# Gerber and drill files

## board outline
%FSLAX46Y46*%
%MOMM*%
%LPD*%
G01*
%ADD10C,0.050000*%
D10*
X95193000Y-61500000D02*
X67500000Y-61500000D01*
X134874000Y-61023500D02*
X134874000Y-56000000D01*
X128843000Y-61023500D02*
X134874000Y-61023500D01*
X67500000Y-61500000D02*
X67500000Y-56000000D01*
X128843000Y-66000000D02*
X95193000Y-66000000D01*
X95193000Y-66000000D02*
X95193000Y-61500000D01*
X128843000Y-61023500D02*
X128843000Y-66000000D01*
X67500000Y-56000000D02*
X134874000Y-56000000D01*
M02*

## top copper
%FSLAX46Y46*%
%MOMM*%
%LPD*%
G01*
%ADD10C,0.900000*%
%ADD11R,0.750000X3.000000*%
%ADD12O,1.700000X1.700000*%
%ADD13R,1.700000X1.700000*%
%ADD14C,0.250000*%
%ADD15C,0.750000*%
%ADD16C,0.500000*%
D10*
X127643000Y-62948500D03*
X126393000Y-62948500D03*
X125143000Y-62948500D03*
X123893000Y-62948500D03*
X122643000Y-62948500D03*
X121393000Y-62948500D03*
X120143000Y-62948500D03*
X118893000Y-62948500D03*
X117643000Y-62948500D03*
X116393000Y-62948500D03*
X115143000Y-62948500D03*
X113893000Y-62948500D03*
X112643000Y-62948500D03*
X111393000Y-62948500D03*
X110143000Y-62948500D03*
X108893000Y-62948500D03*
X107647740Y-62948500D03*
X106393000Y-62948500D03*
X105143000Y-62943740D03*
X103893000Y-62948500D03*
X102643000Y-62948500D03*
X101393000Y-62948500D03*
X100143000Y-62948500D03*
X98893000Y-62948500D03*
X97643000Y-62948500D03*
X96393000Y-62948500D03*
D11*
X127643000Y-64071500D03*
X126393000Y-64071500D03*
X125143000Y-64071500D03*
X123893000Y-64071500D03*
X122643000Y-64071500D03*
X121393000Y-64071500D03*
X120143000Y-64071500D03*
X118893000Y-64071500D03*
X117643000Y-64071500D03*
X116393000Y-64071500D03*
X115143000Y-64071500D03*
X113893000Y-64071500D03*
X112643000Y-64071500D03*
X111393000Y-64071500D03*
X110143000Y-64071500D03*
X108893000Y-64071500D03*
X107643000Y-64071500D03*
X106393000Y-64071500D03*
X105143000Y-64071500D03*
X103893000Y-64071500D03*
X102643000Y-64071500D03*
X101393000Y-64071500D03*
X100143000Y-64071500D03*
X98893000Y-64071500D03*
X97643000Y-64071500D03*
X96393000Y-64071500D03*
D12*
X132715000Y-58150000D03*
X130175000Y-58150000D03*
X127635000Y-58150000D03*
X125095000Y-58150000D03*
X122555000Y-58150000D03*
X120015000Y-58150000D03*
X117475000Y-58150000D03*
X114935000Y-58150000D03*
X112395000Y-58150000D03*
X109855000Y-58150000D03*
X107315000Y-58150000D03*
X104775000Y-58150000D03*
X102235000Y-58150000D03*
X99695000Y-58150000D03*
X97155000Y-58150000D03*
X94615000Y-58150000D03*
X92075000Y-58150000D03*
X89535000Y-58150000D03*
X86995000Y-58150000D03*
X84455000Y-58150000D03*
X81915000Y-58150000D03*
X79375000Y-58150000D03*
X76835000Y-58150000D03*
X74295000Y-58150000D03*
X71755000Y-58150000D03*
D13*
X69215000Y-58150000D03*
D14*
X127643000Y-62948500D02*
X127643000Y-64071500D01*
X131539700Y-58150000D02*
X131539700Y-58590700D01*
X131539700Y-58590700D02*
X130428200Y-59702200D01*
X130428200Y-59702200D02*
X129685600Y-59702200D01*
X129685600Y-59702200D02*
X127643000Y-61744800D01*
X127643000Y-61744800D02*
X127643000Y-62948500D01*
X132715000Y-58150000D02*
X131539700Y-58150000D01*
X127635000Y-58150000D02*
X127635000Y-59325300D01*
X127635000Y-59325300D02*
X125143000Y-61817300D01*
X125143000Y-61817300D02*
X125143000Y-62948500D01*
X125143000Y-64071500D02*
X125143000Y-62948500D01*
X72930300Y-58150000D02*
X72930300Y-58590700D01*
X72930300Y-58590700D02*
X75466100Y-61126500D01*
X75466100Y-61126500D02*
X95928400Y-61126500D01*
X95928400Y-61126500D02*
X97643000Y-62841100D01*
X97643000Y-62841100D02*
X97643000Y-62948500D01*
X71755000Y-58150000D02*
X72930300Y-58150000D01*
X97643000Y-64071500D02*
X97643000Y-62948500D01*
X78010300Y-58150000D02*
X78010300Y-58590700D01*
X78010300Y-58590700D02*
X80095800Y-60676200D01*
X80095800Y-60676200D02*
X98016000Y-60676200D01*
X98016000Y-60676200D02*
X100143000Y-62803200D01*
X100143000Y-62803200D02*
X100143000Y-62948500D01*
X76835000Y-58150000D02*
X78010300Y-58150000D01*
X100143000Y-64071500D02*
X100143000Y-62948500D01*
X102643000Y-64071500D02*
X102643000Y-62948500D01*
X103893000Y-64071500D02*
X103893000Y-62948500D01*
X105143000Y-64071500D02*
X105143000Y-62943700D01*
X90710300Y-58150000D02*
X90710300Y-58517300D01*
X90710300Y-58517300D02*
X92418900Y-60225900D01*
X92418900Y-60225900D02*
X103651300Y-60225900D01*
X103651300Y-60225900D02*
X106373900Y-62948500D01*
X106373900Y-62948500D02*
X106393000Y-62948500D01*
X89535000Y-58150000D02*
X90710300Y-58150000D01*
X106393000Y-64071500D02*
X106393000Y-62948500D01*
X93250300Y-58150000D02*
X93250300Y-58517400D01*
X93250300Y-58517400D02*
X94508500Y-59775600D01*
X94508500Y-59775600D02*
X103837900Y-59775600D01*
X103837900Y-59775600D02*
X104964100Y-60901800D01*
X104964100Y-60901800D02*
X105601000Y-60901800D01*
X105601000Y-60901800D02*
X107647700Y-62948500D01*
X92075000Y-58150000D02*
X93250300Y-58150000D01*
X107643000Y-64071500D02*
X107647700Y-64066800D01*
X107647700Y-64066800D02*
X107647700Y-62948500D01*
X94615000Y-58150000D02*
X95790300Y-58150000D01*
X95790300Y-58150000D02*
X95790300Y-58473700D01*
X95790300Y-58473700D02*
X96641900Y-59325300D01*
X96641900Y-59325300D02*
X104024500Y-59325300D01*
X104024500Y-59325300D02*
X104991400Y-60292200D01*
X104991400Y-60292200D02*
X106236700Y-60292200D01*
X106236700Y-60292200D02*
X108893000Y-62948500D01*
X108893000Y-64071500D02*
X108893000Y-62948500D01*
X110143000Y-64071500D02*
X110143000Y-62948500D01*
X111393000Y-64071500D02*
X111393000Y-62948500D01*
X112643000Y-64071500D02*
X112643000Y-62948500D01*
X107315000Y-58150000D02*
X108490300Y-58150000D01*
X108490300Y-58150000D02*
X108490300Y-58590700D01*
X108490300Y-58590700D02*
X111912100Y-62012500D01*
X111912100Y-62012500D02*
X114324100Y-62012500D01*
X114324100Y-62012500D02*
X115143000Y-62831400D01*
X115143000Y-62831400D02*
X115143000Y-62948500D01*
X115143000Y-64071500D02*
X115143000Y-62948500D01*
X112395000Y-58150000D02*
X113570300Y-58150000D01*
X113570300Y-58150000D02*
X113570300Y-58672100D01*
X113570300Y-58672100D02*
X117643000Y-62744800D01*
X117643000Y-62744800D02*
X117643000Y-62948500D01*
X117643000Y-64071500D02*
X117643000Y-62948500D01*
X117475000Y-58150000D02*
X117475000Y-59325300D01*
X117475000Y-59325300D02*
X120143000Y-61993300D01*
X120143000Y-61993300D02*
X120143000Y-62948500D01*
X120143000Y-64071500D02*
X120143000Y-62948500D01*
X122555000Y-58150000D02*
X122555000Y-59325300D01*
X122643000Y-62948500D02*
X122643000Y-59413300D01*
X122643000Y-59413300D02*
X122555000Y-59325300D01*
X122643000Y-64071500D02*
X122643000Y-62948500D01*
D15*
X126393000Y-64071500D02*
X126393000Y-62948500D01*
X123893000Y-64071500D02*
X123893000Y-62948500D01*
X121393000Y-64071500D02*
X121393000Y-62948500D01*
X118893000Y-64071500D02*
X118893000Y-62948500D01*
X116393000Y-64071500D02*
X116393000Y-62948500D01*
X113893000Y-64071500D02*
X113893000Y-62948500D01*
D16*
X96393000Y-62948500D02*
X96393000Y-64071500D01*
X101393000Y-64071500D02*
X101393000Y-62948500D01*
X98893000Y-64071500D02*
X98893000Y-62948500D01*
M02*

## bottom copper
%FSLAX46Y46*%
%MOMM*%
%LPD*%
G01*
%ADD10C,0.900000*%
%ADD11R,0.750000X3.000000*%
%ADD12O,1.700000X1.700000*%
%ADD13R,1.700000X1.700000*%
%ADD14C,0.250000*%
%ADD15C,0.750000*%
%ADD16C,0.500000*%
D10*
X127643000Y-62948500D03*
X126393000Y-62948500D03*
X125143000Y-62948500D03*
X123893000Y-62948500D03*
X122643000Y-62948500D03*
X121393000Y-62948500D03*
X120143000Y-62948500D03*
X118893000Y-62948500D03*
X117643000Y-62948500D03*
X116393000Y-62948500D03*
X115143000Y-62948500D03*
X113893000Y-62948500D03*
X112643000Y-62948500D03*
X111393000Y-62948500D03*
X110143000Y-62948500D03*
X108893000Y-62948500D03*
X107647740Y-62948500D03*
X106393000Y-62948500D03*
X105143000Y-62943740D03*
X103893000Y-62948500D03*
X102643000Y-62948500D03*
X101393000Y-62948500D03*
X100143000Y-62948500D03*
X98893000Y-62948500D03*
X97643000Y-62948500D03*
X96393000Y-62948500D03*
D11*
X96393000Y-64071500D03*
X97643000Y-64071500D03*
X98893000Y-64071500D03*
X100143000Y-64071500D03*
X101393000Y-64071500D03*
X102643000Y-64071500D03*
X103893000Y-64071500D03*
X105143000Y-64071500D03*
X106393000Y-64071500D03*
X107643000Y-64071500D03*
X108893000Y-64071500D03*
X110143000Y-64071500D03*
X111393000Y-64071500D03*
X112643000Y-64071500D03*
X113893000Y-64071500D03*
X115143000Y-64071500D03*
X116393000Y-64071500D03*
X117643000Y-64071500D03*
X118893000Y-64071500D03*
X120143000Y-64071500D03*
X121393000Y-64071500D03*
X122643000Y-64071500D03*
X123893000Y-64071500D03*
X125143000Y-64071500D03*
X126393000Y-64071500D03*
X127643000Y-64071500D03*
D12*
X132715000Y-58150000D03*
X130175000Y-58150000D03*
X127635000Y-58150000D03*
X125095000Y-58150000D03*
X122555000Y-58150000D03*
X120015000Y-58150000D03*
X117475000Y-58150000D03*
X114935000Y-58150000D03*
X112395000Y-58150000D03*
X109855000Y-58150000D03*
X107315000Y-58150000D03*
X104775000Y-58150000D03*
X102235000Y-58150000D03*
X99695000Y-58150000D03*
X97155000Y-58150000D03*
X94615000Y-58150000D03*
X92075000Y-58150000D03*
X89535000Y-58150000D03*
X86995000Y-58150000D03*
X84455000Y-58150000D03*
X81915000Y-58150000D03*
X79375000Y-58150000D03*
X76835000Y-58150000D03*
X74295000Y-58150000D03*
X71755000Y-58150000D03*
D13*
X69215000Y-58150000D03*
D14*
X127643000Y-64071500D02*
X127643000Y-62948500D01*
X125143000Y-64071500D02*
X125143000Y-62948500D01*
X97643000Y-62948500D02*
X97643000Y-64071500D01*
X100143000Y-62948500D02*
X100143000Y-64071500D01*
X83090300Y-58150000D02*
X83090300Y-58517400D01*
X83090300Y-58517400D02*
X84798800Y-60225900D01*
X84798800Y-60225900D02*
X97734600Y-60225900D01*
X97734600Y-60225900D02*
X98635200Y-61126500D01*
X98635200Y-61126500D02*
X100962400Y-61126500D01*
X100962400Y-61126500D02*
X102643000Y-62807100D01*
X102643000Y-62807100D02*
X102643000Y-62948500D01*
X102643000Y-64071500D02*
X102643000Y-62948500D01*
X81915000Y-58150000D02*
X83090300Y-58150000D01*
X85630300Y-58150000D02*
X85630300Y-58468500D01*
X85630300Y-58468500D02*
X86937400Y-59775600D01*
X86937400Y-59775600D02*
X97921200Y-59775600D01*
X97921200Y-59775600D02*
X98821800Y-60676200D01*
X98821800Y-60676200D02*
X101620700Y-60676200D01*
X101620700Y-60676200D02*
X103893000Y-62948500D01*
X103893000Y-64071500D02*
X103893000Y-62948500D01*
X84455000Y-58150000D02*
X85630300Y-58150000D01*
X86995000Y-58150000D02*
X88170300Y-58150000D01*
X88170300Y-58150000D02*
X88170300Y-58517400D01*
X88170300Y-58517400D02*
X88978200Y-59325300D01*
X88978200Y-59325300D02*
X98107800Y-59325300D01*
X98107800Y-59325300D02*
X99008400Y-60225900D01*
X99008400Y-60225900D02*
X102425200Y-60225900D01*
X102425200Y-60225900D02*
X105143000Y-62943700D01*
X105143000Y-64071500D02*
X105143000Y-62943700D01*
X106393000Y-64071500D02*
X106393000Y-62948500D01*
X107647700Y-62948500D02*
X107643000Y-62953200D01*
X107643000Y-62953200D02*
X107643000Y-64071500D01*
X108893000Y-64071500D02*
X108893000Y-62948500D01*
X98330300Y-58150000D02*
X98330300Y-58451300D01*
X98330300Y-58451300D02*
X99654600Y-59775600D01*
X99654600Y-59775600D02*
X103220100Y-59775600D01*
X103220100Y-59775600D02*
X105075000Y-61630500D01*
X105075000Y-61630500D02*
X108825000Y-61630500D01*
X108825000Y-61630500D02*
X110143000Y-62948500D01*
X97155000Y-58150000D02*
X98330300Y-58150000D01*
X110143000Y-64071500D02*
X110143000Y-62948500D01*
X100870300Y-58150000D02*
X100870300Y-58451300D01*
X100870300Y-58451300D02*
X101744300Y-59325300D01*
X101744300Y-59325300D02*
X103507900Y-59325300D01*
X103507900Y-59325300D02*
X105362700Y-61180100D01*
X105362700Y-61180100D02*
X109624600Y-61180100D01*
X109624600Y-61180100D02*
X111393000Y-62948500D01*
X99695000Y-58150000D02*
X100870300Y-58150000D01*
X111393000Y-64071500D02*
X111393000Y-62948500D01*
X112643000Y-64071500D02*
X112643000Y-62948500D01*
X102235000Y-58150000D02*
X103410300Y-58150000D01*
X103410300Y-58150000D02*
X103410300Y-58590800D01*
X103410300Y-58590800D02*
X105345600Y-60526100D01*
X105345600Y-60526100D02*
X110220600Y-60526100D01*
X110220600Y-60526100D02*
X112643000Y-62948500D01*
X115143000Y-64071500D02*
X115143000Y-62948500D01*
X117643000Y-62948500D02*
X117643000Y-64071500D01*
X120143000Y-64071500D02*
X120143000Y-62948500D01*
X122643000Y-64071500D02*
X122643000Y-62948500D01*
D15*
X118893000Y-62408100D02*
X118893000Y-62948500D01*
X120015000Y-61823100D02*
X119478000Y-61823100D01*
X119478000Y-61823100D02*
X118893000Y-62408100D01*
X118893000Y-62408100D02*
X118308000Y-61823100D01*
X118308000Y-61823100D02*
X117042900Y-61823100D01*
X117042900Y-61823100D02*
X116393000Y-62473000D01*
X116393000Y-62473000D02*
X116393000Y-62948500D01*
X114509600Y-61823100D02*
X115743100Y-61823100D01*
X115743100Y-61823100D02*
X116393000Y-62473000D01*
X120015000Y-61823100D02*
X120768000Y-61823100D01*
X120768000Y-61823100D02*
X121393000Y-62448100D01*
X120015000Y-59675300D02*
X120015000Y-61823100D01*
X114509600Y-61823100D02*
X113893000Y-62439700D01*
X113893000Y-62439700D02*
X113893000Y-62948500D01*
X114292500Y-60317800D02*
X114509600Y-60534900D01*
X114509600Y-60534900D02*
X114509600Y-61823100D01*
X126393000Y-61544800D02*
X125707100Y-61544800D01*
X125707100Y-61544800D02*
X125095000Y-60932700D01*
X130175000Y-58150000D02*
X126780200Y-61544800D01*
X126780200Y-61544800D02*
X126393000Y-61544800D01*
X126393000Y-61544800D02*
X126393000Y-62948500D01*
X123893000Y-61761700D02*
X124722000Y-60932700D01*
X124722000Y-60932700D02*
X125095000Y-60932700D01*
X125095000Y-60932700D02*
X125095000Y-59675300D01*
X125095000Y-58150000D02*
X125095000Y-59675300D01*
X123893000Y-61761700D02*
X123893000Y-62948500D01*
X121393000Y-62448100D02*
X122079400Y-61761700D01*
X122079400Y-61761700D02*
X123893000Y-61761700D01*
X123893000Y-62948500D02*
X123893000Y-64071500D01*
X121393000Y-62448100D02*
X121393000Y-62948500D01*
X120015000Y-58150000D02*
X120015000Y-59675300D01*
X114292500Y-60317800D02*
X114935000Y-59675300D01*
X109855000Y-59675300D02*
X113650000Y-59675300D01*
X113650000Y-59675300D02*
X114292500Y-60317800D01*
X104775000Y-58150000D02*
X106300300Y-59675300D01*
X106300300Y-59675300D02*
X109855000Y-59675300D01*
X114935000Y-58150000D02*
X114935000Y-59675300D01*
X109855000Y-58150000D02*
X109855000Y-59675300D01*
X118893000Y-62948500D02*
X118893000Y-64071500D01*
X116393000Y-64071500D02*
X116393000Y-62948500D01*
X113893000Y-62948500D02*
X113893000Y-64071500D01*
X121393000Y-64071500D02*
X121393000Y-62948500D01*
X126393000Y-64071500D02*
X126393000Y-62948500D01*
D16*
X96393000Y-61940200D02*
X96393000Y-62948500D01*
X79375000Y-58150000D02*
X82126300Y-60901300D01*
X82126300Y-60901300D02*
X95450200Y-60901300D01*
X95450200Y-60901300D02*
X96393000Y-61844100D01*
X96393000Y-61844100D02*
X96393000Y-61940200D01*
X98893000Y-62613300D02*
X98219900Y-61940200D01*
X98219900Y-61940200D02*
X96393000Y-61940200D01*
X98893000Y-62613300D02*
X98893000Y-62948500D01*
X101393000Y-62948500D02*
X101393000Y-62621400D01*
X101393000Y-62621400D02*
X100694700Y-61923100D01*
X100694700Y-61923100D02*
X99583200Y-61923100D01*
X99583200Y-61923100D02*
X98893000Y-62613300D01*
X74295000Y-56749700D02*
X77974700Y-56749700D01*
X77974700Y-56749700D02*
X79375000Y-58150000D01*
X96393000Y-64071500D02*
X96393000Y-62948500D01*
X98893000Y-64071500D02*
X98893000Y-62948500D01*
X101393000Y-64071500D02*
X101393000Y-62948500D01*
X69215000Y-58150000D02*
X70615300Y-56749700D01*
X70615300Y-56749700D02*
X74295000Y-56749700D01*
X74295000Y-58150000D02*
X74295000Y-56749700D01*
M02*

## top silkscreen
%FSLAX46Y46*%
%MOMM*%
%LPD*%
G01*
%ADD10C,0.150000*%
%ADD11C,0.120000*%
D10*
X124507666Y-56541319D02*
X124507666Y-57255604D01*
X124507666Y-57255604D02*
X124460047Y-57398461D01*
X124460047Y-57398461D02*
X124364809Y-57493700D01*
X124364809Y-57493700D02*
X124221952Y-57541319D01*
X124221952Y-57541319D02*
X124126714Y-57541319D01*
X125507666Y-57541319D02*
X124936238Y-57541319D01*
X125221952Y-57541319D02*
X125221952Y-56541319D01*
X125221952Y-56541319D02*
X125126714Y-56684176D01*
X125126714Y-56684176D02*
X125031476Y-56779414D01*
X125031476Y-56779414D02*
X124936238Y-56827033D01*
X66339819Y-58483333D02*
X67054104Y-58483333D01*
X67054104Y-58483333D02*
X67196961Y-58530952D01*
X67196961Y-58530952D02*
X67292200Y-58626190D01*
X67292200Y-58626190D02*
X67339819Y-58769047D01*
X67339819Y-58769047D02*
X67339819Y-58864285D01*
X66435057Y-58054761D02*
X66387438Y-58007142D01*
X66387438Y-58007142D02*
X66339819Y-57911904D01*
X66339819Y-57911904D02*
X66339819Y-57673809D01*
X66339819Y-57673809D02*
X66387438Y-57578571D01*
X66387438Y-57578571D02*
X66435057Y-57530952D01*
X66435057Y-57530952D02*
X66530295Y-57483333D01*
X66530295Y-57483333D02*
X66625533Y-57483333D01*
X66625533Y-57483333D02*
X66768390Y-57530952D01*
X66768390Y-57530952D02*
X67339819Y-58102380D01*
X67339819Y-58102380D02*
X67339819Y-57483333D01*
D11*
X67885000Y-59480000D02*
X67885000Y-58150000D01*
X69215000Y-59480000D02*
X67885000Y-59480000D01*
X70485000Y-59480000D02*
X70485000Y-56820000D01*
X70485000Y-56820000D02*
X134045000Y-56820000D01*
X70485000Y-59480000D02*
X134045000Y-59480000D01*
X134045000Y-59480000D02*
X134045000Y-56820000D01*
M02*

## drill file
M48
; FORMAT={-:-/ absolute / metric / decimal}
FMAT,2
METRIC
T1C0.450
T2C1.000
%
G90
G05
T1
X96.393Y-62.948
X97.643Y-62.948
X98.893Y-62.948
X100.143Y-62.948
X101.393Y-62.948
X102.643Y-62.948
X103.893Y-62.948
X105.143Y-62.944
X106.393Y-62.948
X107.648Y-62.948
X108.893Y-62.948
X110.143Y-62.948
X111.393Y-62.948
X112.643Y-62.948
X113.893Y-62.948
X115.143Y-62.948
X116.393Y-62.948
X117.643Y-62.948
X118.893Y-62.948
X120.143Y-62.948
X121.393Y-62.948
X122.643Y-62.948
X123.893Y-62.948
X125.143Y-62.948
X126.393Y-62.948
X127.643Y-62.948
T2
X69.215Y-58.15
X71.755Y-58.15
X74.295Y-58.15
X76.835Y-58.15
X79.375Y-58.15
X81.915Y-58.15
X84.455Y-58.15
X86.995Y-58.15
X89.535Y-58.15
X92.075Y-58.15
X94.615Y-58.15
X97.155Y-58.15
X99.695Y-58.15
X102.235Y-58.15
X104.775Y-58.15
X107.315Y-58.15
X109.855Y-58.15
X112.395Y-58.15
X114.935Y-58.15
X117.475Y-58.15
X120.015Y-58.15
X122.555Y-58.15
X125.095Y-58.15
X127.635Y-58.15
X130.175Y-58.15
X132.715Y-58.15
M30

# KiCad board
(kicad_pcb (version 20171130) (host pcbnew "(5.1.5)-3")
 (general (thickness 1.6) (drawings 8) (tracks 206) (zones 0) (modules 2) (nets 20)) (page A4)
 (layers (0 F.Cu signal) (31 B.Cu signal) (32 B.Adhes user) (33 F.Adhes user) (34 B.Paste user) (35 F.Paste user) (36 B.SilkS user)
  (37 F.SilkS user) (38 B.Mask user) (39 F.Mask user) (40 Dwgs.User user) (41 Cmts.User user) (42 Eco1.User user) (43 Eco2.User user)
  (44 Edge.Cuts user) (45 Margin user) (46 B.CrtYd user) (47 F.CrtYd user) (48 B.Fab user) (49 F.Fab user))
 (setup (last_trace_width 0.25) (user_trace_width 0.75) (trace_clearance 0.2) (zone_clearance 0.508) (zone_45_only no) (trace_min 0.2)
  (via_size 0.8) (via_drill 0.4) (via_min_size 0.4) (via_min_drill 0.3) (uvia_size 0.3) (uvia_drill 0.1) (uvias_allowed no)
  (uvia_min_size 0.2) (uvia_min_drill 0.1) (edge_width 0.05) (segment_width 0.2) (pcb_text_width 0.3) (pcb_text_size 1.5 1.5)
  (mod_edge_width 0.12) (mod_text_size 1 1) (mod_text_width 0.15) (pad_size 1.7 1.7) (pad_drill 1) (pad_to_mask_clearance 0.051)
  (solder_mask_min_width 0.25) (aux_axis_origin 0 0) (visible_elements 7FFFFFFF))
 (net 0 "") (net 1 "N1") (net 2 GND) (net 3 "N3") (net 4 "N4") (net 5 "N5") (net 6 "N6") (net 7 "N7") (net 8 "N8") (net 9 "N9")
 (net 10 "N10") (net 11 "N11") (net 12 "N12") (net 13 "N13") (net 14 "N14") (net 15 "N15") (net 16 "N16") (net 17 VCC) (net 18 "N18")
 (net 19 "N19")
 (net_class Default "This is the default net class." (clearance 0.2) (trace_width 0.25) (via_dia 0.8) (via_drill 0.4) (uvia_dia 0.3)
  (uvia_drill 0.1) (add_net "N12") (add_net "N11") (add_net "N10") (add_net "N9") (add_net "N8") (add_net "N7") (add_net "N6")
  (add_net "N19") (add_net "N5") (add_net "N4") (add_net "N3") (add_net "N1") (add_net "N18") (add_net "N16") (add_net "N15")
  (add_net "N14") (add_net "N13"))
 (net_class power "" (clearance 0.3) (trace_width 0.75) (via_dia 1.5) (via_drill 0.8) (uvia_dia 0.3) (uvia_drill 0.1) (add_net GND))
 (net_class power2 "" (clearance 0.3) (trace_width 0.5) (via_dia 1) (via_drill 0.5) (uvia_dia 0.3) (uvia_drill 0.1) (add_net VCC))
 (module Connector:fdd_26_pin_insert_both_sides (layer F.Cu) (at 96.393 64.1985)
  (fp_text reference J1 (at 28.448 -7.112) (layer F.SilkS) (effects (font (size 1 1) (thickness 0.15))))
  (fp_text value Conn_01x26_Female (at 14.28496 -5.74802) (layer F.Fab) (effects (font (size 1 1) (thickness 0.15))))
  (pad 26 thru_hole circle (at 31.25 -1.25) (size 0.9 0.9) (drill 0.45) (layers *.Cu *.Mask) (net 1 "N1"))
  (pad 25 thru_hole circle (at 30 -1.25) (size 0.9 0.9) (drill 0.45) (layers *.Cu *.Mask) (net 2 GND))
  (pad 24 thru_hole circle (at 28.75 -1.25) (size 0.9 0.9) (drill 0.45) (layers *.Cu *.Mask) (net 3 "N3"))
  (pad 23 thru_hole circle (at 27.5 -1.25) (size 0.9 0.9) (drill 0.45) (layers *.Cu *.Mask) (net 2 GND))
  (pad 22 thru_hole circle (at 26.25 -1.25) (size 0.9 0.9) (drill 0.45) (layers *.Cu *.Mask) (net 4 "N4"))
  (pad 21 thru_hole circle (at 25 -1.25) (size 0.9 0.9) (drill 0.45) (layers *.Cu *.Mask) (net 2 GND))
  (pad 20 thru_hole circle (at 23.75 -1.25) (size 0.9 0.9) (drill 0.45) (layers *.Cu *.Mask) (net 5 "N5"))
  (pad 19 thru_hole circle (at 22.5 -1.25) (size 0.9 0.9) (drill 0.45) (layers *.Cu *.Mask) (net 2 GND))
  (pad 18 thru_hole circle (at 21.25 -1.25) (size 0.9 0.9) (drill 0.45) (layers *.Cu *.Mask) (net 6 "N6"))
  (pad 17 thru_hole circle (at 20 -1.25) (size 0.9 0.9) (drill 0.45) (layers *.Cu *.Mask) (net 2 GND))
  (pad 16 thru_hole circle (at 18.75 -1.25) (size 0.9 0.9) (drill 0.45) (layers *.Cu *.Mask) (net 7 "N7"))
  (pad 15 thru_hole circle (at 17.5 -1.25 90) (size 0.9 0.9) (drill 0.45) (layers *.Cu *.Mask) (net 2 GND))
  (pad 14 thru_hole circle (at 16.25 -1.25) (size 0.9 0.9) (drill 0.45) (layers *.Cu *.Mask) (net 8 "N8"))
  (pad 13 thru_hole circle (at 15 -1.25) (size 0.9 0.9) (drill 0.45) (layers *.Cu *.Mask) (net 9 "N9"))
  (pad 12 thru_hole circle (at 13.75 -1.25) (size 0.9 0.9) (drill 0.45) (layers *.Cu *.Mask) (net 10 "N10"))
  (pad 11 thru_hole circle (at 12.5 -1.25) (size 0.9 0.9) (drill 0.45) (layers *.Cu *.Mask) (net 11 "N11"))
  (pad 10 thru_hole circle (at 11.25474 -1.25) (size 0.9 0.9) (drill 0.45) (layers *.Cu *.Mask) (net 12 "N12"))
  (pad 9 thru_hole circle (at 10 -1.25) (size 0.9 0.9) (drill 0.45) (layers *.Cu *.Mask) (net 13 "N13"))
  (pad 8 thru_hole circle (at 8.75 -1.25476) (size 0.9 0.9) (drill 0.45) (layers *.Cu *.Mask) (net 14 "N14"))
  (pad 7 thru_hole circle (at 7.5 -1.25) (size 0.9 0.9) (drill 0.45) (layers *.Cu *.Mask) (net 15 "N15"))
  (pad 6 thru_hole circle (at 6.25 -1.25) (size 0.9 0.9) (drill 0.45) (layers *.Cu *.Mask) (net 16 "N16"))
  (pad 5 thru_hole circle (at 5 -1.25) (size 0.9 0.9) (drill 0.45) (layers *.Cu *.Mask) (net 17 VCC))
  (pad 4 thru_hole circle (at 3.75 -1.25) (size 0.9 0.9) (drill 0.45) (layers *.Cu *.Mask) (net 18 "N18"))
  (pad 3 thru_hole circle (at 2.5 -1.25) (size 0.9 0.9) (drill 0.45) (layers *.Cu *.Mask) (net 17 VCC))
  (pad 2 thru_hole circle (at 1.25 -1.25 90) (size 0.9 0.9) (drill 0.45) (layers *.Cu *.Mask) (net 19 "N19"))
  (pad 1 thru_hole circle (at 0 -1.25) (size 0.9 0.9) (drill 0.45) (layers *.Cu *.Mask) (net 17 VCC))
  (pad 26 connect rect (at 31.25 -0.127) (size 0.75 3) (layers F.Cu B.Mask) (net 1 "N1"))
  (pad 25 connect rect (at 30 -0.127) (size 0.75 3) (layers F.Cu B.Mask) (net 2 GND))
  (pad 24 connect rect (at 28.75 -0.127) (size 0.75 3) (layers F.Cu B.Mask) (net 3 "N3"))
  (pad 23 connect rect (at 27.5 -0.127) (size 0.75 3) (layers F.Cu B.Mask) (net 2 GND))
  (pad 22 connect rect (at 26.25 -0.127) (size 0.75 3) (layers F.Cu B.Mask) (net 4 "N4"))
  (pad 21 connect rect (at 25 -0.127) (size 0.75 3) (layers F.Cu B.Mask) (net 2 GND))
  (pad 20 connect rect (at 23.75 -0.127) (size 0.75 3) (layers F.Cu B.Mask) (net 5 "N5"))
  (pad 19 connect rect (at 22.5 -0.127) (size 0.75 3) (layers F.Cu B.Mask) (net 2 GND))
  (pad 18 connect rect (at 21.25 -0.127) (size 0.75 3) (layers F.Cu B.Mask) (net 6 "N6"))
  (pad 17 connect rect (at 20 -0.127) (size 0.75 3) (layers F.Cu B.Mask) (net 2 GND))
  (pad 16 connect rect (at 18.75 -0.127) (size 0.75 3) (layers F.Cu B.Mask) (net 7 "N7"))
  (pad 15 connect rect (at 17.5 -0.127) (size 0.75 3) (layers F.Cu B.Mask) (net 2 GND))
  (pad 14 connect rect (at 16.25 -0.127) (size 0.75 3) (layers F.Cu B.Mask) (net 8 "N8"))
  (pad 13 connect rect (at 15 -0.127) (size 0.75 3) (layers F.Cu B.Mask) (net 9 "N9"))
  (pad 12 connect rect (at 13.75 -0.127) (size 0.75 3) (layers F.Cu B.Mask) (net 10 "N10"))
  (pad 11 connect rect (at 12.5 -0.127) (size 0.75 3) (layers F.Cu B.Mask) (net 11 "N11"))
  (pad 10 connect rect (at 11.25 -0.127) (size 0.75 3) (layers F.Cu B.Mask) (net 12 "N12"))
  (pad 9 connect rect (at 10 -0.127) (size 0.75 3) (layers F.Cu B.Mask) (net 13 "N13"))
  (pad 8 connect rect (at 8.75 -0.127) (size 0.75 3) (layers F.Cu B.Mask) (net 14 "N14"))
  (pad 7 connect rect (at 7.5 -0.127) (size 0.75 3) (layers F.Cu B.Mask) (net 15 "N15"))
  (pad 6 connect rect (at 6.25 -0.127) (size 0.75 3) (layers F.Cu B.Mask) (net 16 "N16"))
  (pad 5 connect rect (at 5 -0.127) (size 0.75 3) (layers F.Cu B.Mask) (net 17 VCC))
  (pad 4 connect rect (at 3.75 -0.127) (size 0.75 3) (layers F.Cu B.Mask) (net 18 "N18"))
  (pad 3 connect rect (at 2.5 -0.127) (size 0.75 3) (layers F.Cu B.Mask) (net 17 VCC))
  (pad 2 connect rect (at 1.25 -0.127) (size 0.75 3) (layers F.Cu B.Mask) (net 19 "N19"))
  (pad 1 connect rect (at 0 -0.127) (size 0.75 3) (layers F.Cu B.Mask) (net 17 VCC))
  (pad 1 connect rect (at 0 -0.127) (size 0.75 3) (layers B.Cu B.Mask) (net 17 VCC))
  (pad 2 connect rect (at 1.25 -0.127) (size 0.75 3) (layers B.Cu B.Mask) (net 19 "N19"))
  (pad 3 connect rect (at 2.5 -0.127) (size 0.75 3) (layers B.Cu B.Mask) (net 17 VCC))
  (pad 4 connect rect (at 3.75 -0.127) (size 0.75 3) (layers B.Cu B.Mask) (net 18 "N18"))
  (pad 5 connect rect (at 5 -0.127) (size 0.75 3) (layers B.Cu B.Mask) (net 17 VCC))
  (pad 6 connect rect (at 6.25 -0.127) (size 0.75 3) (layers B.Cu B.Mask) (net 16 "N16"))
  (pad 7 connect rect (at 7.5 -0.127) (size 0.75 3) (layers B.Cu B.Mask) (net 15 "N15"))
  (pad 8 connect rect (at 8.75 -0.127) (size 0.75 3) (layers B.Cu B.Mask) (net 14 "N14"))
  (pad 9 connect rect (at 10 -0.127) (size 0.75 3) (layers B.Cu B.Mask) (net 13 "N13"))
  (pad 10 connect rect (at 11.25 -0.127) (size 0.75 3) (layers B.Cu B.Mask) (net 12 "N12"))
  (pad 11 connect rect (at 12.5 -0.127) (size 0.75 3) (layers B.Cu B.Mask) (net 11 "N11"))
  (pad 12 connect rect (at 13.75 -0.127) (size 0.75 3) (layers B.Cu B.Mask) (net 10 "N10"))
  (pad 13 connect rect (at 15 -0.127) (size 0.75 3) (layers B.Cu B.Mask) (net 9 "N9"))
  (pad 14 connect rect (at 16.25 -0.127) (size 0.75 3) (layers B.Cu B.Mask) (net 8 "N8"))
  (pad 15 connect rect (at 17.5 -0.127) (size 0.75 3) (layers B.Cu B.Mask) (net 2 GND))
  (pad 16 connect rect (at 18.75 -0.127) (size 0.75 3) (layers B.Cu B.Mask) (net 7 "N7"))
  (pad 17 connect rect (at 20 -0.127) (size 0.75 3) (layers B.Cu B.Mask) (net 2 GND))
  (pad 18 connect rect (at 21.25 -0.127) (size 0.75 3) (layers B.Cu B.Mask) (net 6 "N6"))
  (pad 19 connect rect (at 22.5 -0.127) (size 0.75 3) (layers B.Cu B.Mask) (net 2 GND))
  (pad 20 connect rect (at 23.75 -0.127) (size 0.75 3) (layers B.Cu B.Mask) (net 5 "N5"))
  (pad 21 connect rect (at 25 -0.127) (size 0.75 3) (layers B.Cu B.Mask) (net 2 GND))
  (pad 22 connect rect (at 26.25 -0.127) (size 0.75 3) (layers B.Cu B.Mask) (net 4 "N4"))
  (pad 23 connect rect (at 27.5 -0.127) (size 0.75 3) (layers B.Cu B.Mask) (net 2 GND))
  (pad 24 connect rect (at 28.75 -0.127) (size 0.75 3) (layers B.Cu B.Mask) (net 3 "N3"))
  (pad 25 connect rect (at 30 -0.127) (size 0.75 3) (layers B.Cu B.Mask) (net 2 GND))
  (pad 26 connect rect (at 31.25 -0.127) (size 0.75 3) (layers B.Cu B.Mask) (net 1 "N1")))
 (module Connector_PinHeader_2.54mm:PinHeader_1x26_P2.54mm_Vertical (layer F.Cu) (at 69.215 58.15 90)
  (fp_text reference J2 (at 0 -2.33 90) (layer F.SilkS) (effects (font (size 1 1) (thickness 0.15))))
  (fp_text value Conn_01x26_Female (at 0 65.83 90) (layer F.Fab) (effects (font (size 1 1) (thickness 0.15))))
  (fp_line (start -1.33 -1.33) (end 0 -1.33) (layer F.SilkS) (width 0.12))
  (fp_line (start -1.33 0) (end -1.33 -1.33) (layer F.SilkS) (width 0.12))
  (fp_line (start -1.33 1.27) (end 1.33 1.27) (layer F.SilkS) (width 0.12))
  (fp_line (start 1.33 1.27) (end 1.33 64.83) (layer F.SilkS) (width 0.12))
  (fp_line (start -1.33 1.27) (end -1.33 64.83) (layer F.SilkS) (width 0.12))
  (fp_line (start -1.33 64.83) (end 1.33 64.83) (layer F.SilkS) (width 0.12))
  (pad 26 thru_hole oval (at 0 63.5 90) (size 1.7 1.7) (drill 1) (layers *.Cu *.Mask) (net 1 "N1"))
  (pad 25 thru_hole oval (at 0 60.96 90) (size 1.7 1.7) (drill 1) (layers *.Cu *.Mask) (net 2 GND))
  (pad 24 thru_hole oval (at 0 58.42 90) (size 1.7 1.7) (drill 1) (layers *.Cu *.Mask) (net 3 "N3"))
  (pad 23 thru_hole oval (at 0 55.88 90) (size 1.7 1.7) (drill 1) (layers *.Cu *.Mask) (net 2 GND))
  (pad 22 thru_hole oval (at 0 53.34 90) (size 1.7 1.7) (drill 1) (layers *.Cu *.Mask) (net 4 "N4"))
  (pad 21 thru_hole oval (at 0 50.8 90) (size 1.7 1.7) (drill 1) (layers *.Cu *.Mask) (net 2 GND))
  (pad 20 thru_hole oval (at 0 48.26 90) (size 1.7 1.7) (drill 1) (layers *.Cu *.Mask) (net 5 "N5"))
  (pad 19 thru_hole oval (at 0 45.72 90) (size 1.7 1.7) (drill 1) (layers *.Cu *.Mask) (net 2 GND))
  (pad 18 thru_hole oval (at 0 43.18 90) (size 1.7 1.7) (drill 1) (layers *.Cu *.Mask) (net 6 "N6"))
  (pad 17 thru_hole oval (at 0 40.64 90) (size 1.7 1.7) (drill 1) (layers *.Cu *.Mask) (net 2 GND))
  (pad 16 thru_hole oval (at 0 38.1 90) (size 1.7 1.7) (drill 1) (layers *.Cu *.Mask) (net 7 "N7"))
  (pad 15 thru_hole oval (at 0 35.56 90) (size 1.7 1.7) (drill 1) (layers *.Cu *.Mask) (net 2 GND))
  (pad 14 thru_hole oval (at 0 33.02 90) (size 1.7 1.7) (drill 1) (layers *.Cu *.Mask) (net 8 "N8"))
  (pad 13 thru_hole oval (at 0 30.48 90) (size 1.7 1.7) (drill 1) (layers *.Cu *.Mask) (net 9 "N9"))
  (pad 12 thru_hole oval (at 0 27.94 90) (size 1.7 1.7) (drill 1) (layers *.Cu *.Mask) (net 10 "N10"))
  (pad 11 thru_hole oval (at 0 25.4 90) (size 1.7 1.7) (drill 1) (layers *.Cu *.Mask) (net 11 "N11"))
  (pad 10 thru_hole oval (at 0 22.86 90) (size 1.7 1.7) (drill 1) (layers *.Cu *.Mask) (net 12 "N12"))
  (pad 9 thru_hole oval (at 0 20.32 90) (size 1.7 1.7) (drill 1) (layers *.Cu *.Mask) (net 13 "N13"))
  (pad 8 thru_hole oval (at 0 17.78 90) (size 1.7 1.7) (drill 1) (layers *.Cu *.Mask) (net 14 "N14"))
  (pad 7 thru_hole oval (at 0 15.24 90) (size 1.7 1.7) (drill 1) (layers *.Cu *.Mask) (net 15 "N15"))
  (pad 6 thru_hole oval (at 0 12.7 90) (size 1.7 1.7) (drill 1) (layers *.Cu *.Mask) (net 16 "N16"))
  (pad 5 thru_hole oval (at 0 10.16 90) (size 1.7 1.7) (drill 1) (layers *.Cu *.Mask) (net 17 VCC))
  (pad 4 thru_hole oval (at 0 7.62 90) (size 1.7 1.7) (drill 1) (layers *.Cu *.Mask) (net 18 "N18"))
  (pad 3 thru_hole oval (at 0 5.08 90) (size 1.7 1.7) (drill 1) (layers *.Cu *.Mask) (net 17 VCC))
  (pad 2 thru_hole oval (at 0 2.54 90) (size 1.7 1.7) (drill 1) (layers *.Cu *.Mask) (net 19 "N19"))
  (pad 1 thru_hole rect (at 0 0 90) (size 1.7 1.7) (drill 1) (layers *.Cu *.Mask) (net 17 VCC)))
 (gr_line (start 95.193 61.5) (end 67.5 61.5) (layer Edge.Cuts) (width 0.05))
 (gr_line (start 134.874 61.0235) (end 134.874 56) (layer Edge.Cuts) (width 0.05))
 (gr_line (start 128.843 61.0235) (end 134.874 61.0235) (layer Edge.Cuts) (width 0.05))
 (gr_line (start 67.5 61.5) (end 67.5 56) (layer Edge.Cuts) (width 0.05))
 (gr_line (start 128.843 66) (end 95.193 66) (layer Edge.Cuts) (width 0.05))
 (gr_line (start 95.193 66) (end 95.193 61.5) (layer Edge.Cuts) (width 0.05))
 (gr_line (start 128.843 61.0235) (end 128.843 66) (layer Edge.Cuts) (width 0.05))
 (gr_line (start 67.5 56) (end 134.874 56) (layer Edge.Cuts) (width 0.05))
 (segment (start 127.643 62.9485) (end 127.643 64.0715) (width 0.25) (layer F.Cu) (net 1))
 (segment (start 131.5397 58.15) (end 131.5397 58.5907) (width 0.25) (layer F.Cu) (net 1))
 (segment (start 131.5397 58.5907) (end 130.4282 59.7022) (width 0.25) (layer F.Cu) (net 1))
 (segment (start 130.4282 59.7022) (end 129.6856 59.7022) (width 0.25) (layer F.Cu) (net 1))
 (segment (start 129.6856 59.7022) (end 127.643 61.7448) (width 0.25) (layer F.Cu) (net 1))
 (segment (start 127.643 61.7448) (end 127.643 62.9485) (width 0.25) (layer F.Cu) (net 1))
 (segment (start 127.643 64.0715) (end 127.643 62.9485) (width 0.25) (layer B.Cu) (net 1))
 (segment (start 132.715 58.15) (end 131.5397 58.15) (width 0.25) (layer F.Cu) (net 1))
 (segment (start 127.635 58.15) (end 127.635 59.3253) (width 0.25) (layer F.Cu) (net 3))
 (segment (start 127.635 59.3253) (end 125.143 61.8173) (width 0.25) (layer F.Cu) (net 3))
 (segment (start 125.143 61.8173) (end 125.143 62.9485) (width 0.25) (layer F.Cu) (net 3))
 (segment (start 125.143 64.0715) (end 125.143 62.9485) (width 0.25) (layer B.Cu) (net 3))
 (segment (start 125.143 64.0715) (end 125.143 62.9485) (width 0.25) (layer F.Cu) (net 3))
 (segment (start 72.9303 58.15) (end 72.9303 58.5907) (width 0.25) (layer F.Cu) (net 19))
 (segment (start 72.9303 58.5907) (end 75.4661 61.1265) (width 0.25) (layer F.Cu) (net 19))
 (segment (start 75.4661 61.1265) (end 95.9284 61.1265) (width 0.25) (layer F.Cu) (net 19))
 (segment (start 95.9284 61.1265) (end 97.643 62.8411) (width 0.25) (layer F.Cu) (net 19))
 (segment (start 97.643 62.8411) (end 97.643 62.9485) (width 0.25) (layer F.Cu) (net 19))
 (segment (start 71.755 58.15) (end 72.9303 58.15) (width 0.25) (layer F.Cu) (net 19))
 (segment (start 97.643 62.9485) (end 97.643 64.0715) (width 0.25) (layer B.Cu) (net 19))
 (segment (start 97.643 64.0715) (end 97.643 62.9485) (width 0.25) (layer F.Cu) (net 19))
 (segment (start 78.0103 58.15) (end 78.0103 58.5907) (width 0.25) (layer F.Cu) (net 18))
 (segment (start 78.0103 58.5907) (end 80.0958 60.6762) (width 0.25) (layer F.Cu) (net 18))
 (segment (start 80.0958 60.6762) (end 98.016 60.6762) (width 0.25) (layer F.Cu) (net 18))
 (segment (start 98.016 60.6762) (end 100.143 62.8032) (width 0.25) (layer F.Cu) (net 18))
 (segment (start 100.143 62.8032) (end 100.143 62.9485) (width 0.25) (layer F.Cu) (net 18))
 (segment (start 76.835 58.15) (end 78.0103 58.15) (width 0.25) (layer F.Cu) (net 18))
 (segment (start 100.143 62.9485) (end 100.143 64.0715) (width 0.25) (layer B.Cu) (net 18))
 (segment (start 100.143 64.0715) (end 100.143 62.9485) (width 0.25) (layer F.Cu) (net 18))
 (segment (start 83.0903 58.15) (end 83.0903 58.5174) (width 0.25) (layer B.Cu) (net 16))
 (segment (start 83.0903 58.5174) (end 84.7988 60.2259) (width 0.25) (layer B.Cu) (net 16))
 (segment (start 84.7988 60.2259) (end 97.7346 60.2259) (width 0.25) (layer B.Cu) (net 16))
 (segment (start 97.7346 60.2259) (end 98.6352 61.1265) (width 0.25) (layer B.Cu) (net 16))
 (segment (start 98.6352 61.1265) (end 100.9624 61.1265) (width 0.25) (layer B.Cu) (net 16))
 (segment (start 100.9624 61.1265) (end 102.643 62.8071) (width 0.25) (layer B.Cu) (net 16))
 (segment (start 102.643 62.8071) (end 102.643 62.9485) (width 0.25) (layer B.Cu) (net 16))
 (segment (start 102.643 64.0715) (end 102.643 62.9485) (width 0.25) (layer F.Cu) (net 16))
 (segment (start 102.643 64.0715) (end 102.643 62.9485) (width 0.25) (layer B.Cu) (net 16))
 (segment (start 81.915 58.15) (end 83.0903 58.15) (width 0.25) (layer B.Cu) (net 16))
 (segment (start 85.6303 58.15) (end 85.6303 58.4685) (width 0.25) (layer B.Cu) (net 15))
 (segment (start 85.6303 58.4685) (end 86.9374 59.7756) (width 0.25) (layer B.Cu) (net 15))
 (segment (start 86.9374 59.7756) (end 97.9212 59.7756) (width 0.25) (layer B.Cu) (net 15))
 (segment (start 97.9212 59.7756) (end 98.8218 60.6762) (width 0.25) (layer B.Cu) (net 15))
 (segment (start 98.8218 60.6762) (end 101.6207 60.6762) (width 0.25) (layer B.Cu) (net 15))
 (segment (start 101.6207 60.6762) (end 103.893 62.9485) (width 0.25) (layer B.Cu) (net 15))
 (segment (start 103.893 64.0715) (end 103.893 62.9485) (width 0.25) (layer F.Cu) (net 15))
 (segment (start 103.893 64.0715) (end 103.893 62.9485) (width 0.25) (layer B.Cu) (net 15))
 (segment (start 84.455 58.15) (end 85.6303 58.15) (width 0.25) (layer B.Cu) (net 15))
 (segment (start 86.995 58.15) (end 88.1703 58.15) (width 0.25) (layer B.Cu) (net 14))
 (segment (start 88.1703 58.15) (end 88.1703 58.5174) (width 0.25) (layer B.Cu) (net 14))
 (segment (start 88.1703 58.5174) (end 88.9782 59.3253) (width 0.25) (layer B.Cu) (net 14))
 (segment (start 88.9782 59.3253) (end 98.1078 59.3253) (width 0.25) (layer B.Cu) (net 14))
 (segment (start 98.1078 59.3253) (end 99.0084 60.2259) (width 0.25) (layer B.Cu) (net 14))
 (segment (start 99.0084 60.2259) (end 102.4252 60.2259) (width 0.25) (layer B.Cu) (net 14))
 (segment (start 102.4252 60.2259) (end 105.143 62.9437) (width 0.25) (layer B.Cu) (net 14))
 (segment (start 105.143 64.0715) (end 105.143 62.9437) (width 0.25) (layer F.Cu) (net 14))
 (segment (start 105.143 64.0715) (end 105.143 62.9437) (width 0.25) (layer B.Cu) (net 14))
 (segment (start 90.7103 58.15) (end 90.7103 58.5173) (width 0.25) (layer F.Cu) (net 13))
 (segment (start 90.7103 58.5173) (end 92.4189 60.2259) (width 0.25) (layer F.Cu) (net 13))
 (segment (start 92.4189 60.2259) (end 103.6513 60.2259) (width 0.25) (layer F.Cu) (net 13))
 (segment (start 103.6513 60.2259) (end 106.3739 62.9485) (width 0.25) (layer F.Cu) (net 13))
 (segment (start 106.3739 62.9485) (end 106.393 62.9485) (width 0.25) (layer F.Cu) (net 13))
 (segment (start 89.535 58.15) (end 90.7103 58.15) (width 0.25) (layer F.Cu) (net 13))
 (segment (start 106.393 64.0715) (end 106.393 62.9485) (width 0.25) (layer B.Cu) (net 13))
 (segment (start 106.393 64.0715) (end 106.393 62.9485) (width 0.25) (layer F.Cu) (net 13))
 (segment (start 93.2503 58.15) (end 93.2503 58.5174) (width 0.25) (layer F.Cu) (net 12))
 (segment (start 93.2503 58.5174) (end 94.5085 59.7756) (width 0.25) (layer F.Cu) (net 12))
 (segment (start 94.5085 59.7756) (end 103.8379 59.7756) (width 0.25) (layer F.Cu) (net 12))
 (segment (start 103.8379 59.7756) (end 104.9641 60.9018) (width 0.25) (layer F.Cu) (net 12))
 (segment (start 104.9641 60.9018) (end 105.601 60.9018) (width 0.25) (layer F.Cu) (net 12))
 (segment (start 105.601 60.9018) (end 107.6477 62.9485) (width 0.25) (layer F.Cu) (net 12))
 (segment (start 92.075 58.15) (end 93.2503 58.15) (width 0.25) (layer F.Cu) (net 12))
 (segment (start 107.6477 62.9485) (end 107.643 62.9532) (width 0.25) (layer B.Cu) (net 12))
 (segment (start 107.643 62.9532) (end 107.643 64.0715) (width 0.25) (layer B.Cu) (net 12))
 (segment (start 107.643 64.0715) (end 107.6477 64.0668) (width 0.25) (layer F.Cu) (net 12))
 (segment (start 107.6477 64.0668) (end 107.6477 62.9485) (width 0.25) (layer F.Cu) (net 12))
 (segment (start 94.615 58.15) (end 95.7903 58.15) (width 0.25) (layer F.Cu) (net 11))
 (segment (start 95.7903 58.15) (end 95.7903 58.4737) (width 0.25) (layer F.Cu) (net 11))
 (segment (start 95.7903 58.4737) (end 96.6419 59.3253) (width 0.25) (layer F.Cu) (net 11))
 (segment (start 96.6419 59.3253) (end 104.0245 59.3253) (width 0.25) (layer F.Cu) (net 11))
 (segment (start 104.0245 59.3253) (end 104.9914 60.2922) (width 0.25) (layer F.Cu) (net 11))
 (segment (start 104.9914 60.2922) (end 106.2367 60.2922) (width 0.25) (layer F.Cu) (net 11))
 (segment (start 106.2367 60.2922) (end 108.893 62.9485) (width 0.25) (layer F.Cu) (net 11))
 (segment (start 108.893 64.0715) (end 108.893 62.9485) (width 0.25) (layer B.Cu) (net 11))
 (segment (start 108.893 64.0715) (end 108.893 62.9485) (width 0.25) (layer F.Cu) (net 11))
 (segment (start 98.3303 58.15) (end 98.3303 58.4513) (width 0.25) (layer B.Cu) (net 10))
 (segment (start 98.3303 58.4513) (end 99.6546 59.7756) (width 0.25) (layer B.Cu) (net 10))
 (segment (start 99.6546 59.7756) (end 103.2201 59.7756) (width 0.25) (layer B.Cu) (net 10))
 (segment (start 103.2201 59.7756) (end 105.075 61.6305) (width 0.25) (layer B.Cu) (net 10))
 (segment (start 105.075 61.6305) (end 108.825 61.6305) (width 0.25) (layer B.Cu) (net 10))
 (segment (start 108.825 61.6305) (end 110.143 62.9485) (width 0.25) (layer B.Cu) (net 10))
 (segment (start 97.155 58.15) (end 98.3303 58.15) (width 0.25) (layer B.Cu) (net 10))
 (segment (start 110.143 64.0715) (end 110.143 62.9485) (width 0.25) (layer B.Cu) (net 10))
 (segment (start 110.143 64.0715) (end 110.143 62.9485) (width 0.25) (layer F.Cu) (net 10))
 (segment (start 100.8703 58.15) (end 100.8703 58.4513) (width 0.25) (layer B.Cu) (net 9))
 (segment (start 100.8703 58.4513) (end 101.7443 59.3253) (width 0.25) (layer B.Cu) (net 9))
 (segment (start 101.7443 59.3253) (end 103.5079 59.3253) (width 0.25) (layer B.Cu) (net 9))
 (segment (start 103.5079 59.3253) (end 105.3627 61.1801) (width 0.25) (layer B.Cu) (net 9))
 (segment (start 105.3627 61.1801) (end 109.6246 61.1801) (width 0.25) (layer B.Cu) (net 9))
 (segment (start 109.6246 61.1801) (end 111.393 62.9485) (width 0.25) (layer B.Cu) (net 9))
 (segment (start 99.695 58.15) (end 100.8703 58.15) (width 0.25) (layer B.Cu) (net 9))
 (segment (start 111.393 64.0715) (end 111.393 62.9485) (width 0.25) (layer B.Cu) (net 9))
 (segment (start 111.393 64.0715) (end 111.393 62.9485) (width 0.25) (layer F.Cu) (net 9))
 (segment (start 112.643 64.0715) (end 112.643 62.9485) (width 0.25) (layer B.Cu) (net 8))
 (segment (start 102.235 58.15) (end 103.4103 58.15) (width 0.25) (layer B.Cu) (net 8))
 (segment (start 103.4103 58.15) (end 103.4103 58.5908) (width 0.25) (layer B.Cu) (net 8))
 (segment (start 103.4103 58.5908) (end 105.3456 60.5261) (width 0.25) (layer B.Cu) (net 8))
 (segment (start 105.3456 60.5261) (end 110.2206 60.5261) (width 0.25) (layer B.Cu) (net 8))
 (segment (start 110.2206 60.5261) (end 112.643 62.9485) (width 0.25) (layer B.Cu) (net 8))
 (segment (start 112.643 64.0715) (end 112.643 62.9485) (width 0.25) (layer F.Cu) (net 8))
 (segment (start 107.315 58.15) (end 108.4903 58.15) (width 0.25) (layer F.Cu) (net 7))
 (segment (start 108.4903 58.15) (end 108.4903 58.5907) (width 0.25) (layer F.Cu) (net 7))
 (segment (start 108.4903 58.5907) (end 111.9121 62.0125) (width 0.25) (layer F.Cu) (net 7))
 (segment (start 111.9121 62.0125) (end 114.3241 62.0125) (width 0.25) (layer F.Cu) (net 7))
 (segment (start 114.3241 62.0125) (end 115.143 62.8314) (width 0.25) (layer F.Cu) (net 7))
 (segment (start 115.143 62.8314) (end 115.143 62.9485) (width 0.25) (layer F.Cu) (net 7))
 (segment (start 115.143 64.0715) (end 115.143 62.9485) (width 0.25) (layer F.Cu) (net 7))
 (segment (start 115.143 64.0715) (end 115.143 62.9485) (width 0.25) (layer B.Cu) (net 7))
 (segment (start 112.395 58.15) (end 113.5703 58.15) (width 0.25) (layer F.Cu) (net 6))
 (segment (start 113.5703 58.15) (end 113.5703 58.6721) (width 0.25) (layer F.Cu) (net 6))
 (segment (start 113.5703 58.6721) (end 117.643 62.7448) (width 0.25) (layer F.Cu) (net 6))
 (segment (start 117.643 62.7448) (end 117.643 62.9485) (width 0.25) (layer F.Cu) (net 6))
 (segment (start 117.643 62.9485) (end 117.643 64.0715) (width 0.25) (layer B.Cu) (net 6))
 (segment (start 117.643 64.0715) (end 117.643 62.9485) (width 0.25) (layer F.Cu) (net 6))
 (segment (start 117.475 58.15) (end 117.475 59.3253) (width 0.25) (layer F.Cu) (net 5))
 (segment (start 117.475 59.3253) (end 120.143 61.9933) (width 0.25) (layer F.Cu) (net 5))
 (segment (start 120.143 61.9933) (end 120.143 62.9485) (width 0.25) (layer F.Cu) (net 5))
 (segment (start 120.143 64.0715) (end 120.143 62.9485) (width 0.25) (layer F.Cu) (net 5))
 (segment (start 120.143 64.0715) (end 120.143 62.9485) (width 0.25) (layer B.Cu) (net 5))
 (segment (start 122.555 58.15) (end 122.555 59.3253) (width 0.25) (layer F.Cu) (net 4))
 (segment (start 122.643 62.9485) (end 122.643 59.4133) (width 0.25) (layer F.Cu) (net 4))
 (segment (start 122.643 59.4133) (end 122.555 59.3253) (width 0.25) (layer F.Cu) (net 4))
 (segment (start 122.643 64.0715) (end 122.643 62.9485) (width 0.25) (layer F.Cu) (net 4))
 (segment (start 122.643 64.0715) (end 122.643 62.9485) (width 0.25) (layer B.Cu) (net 4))
 (segment (start 118.893 62.4081) (end 118.893 62.9485) (width 0.75) (layer B.Cu) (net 2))
 (segment (start 120.015 61.8231) (end 119.478 61.8231) (width 0.75) (layer B.Cu) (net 2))
 (segment (start 119.478 61.8231) (end 118.893 62.4081) (width 0.75) (layer B.Cu) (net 2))
 (segment (start 118.893 62.4081) (end 118.308 61.8231) (width 0.75) (layer B.Cu) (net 2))
 (segment (start 118.308 61.8231) (end 117.0429 61.8231) (width 0.75) (layer B.Cu) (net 2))
 (segment (start 117.0429 61.8231) (end 116.393 62.473) (width 0.75) (layer B.Cu) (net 2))
 (segment (start 116.393 62.473) (end 116.393 62.9485) (width 0.75) (layer B.Cu) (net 2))
 (segment (start 114.5096 61.8231) (end 115.7431 61.8231) (width 0.75) (layer B.Cu) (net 2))
 (segment (start 115.7431 61.8231) (end 116.393 62.473) (width 0.75) (layer B.Cu) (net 2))
 (segment (start 120.015 61.8231) (end 120.768 61.8231) (width 0.75) (layer B.Cu) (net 2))
 (segment (start 120.768 61.8231) (end 121.393 62.4481) (width 0.75) (layer B.Cu) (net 2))
 (segment (start 120.015 59.6753) (end 120.015 61.8231) (width 0.75) (layer B.Cu) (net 2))
 (segment (start 114.5096 61.8231) (end 113.893 62.4397) (width 0.75) (layer B.Cu) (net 2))
 (segment (start 113.893 62.4397) (end 113.893 62.9485) (width 0.75) (layer B.Cu) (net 2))
 (segment (start 114.2925 60.3178) (end 114.5096 60.5349) (width 0.75) (layer B.Cu) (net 2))
 (segment (start 114.5096 60.5349) (end 114.5096 61.8231) (width 0.75) (layer B.Cu) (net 2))
 (segment (start 126.393 61.5448) (end 125.7071 61.5448) (width 0.75) (layer B.Cu) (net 2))
 (segment (start 125.7071 61.5448) (end 125.095 60.9327) (width 0.75) (layer B.Cu) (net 2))
 (segment (start 130.175 58.15) (end 126.7802 61.5448) (width 0.75) (layer B.Cu) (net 2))
 (segment (start 126.7802 61.5448) (end 126.393 61.5448) (width 0.75) (layer B.Cu) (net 2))
 (segment (start 126.393 61.5448) (end 126.393 62.9485) (width 0.75) (layer B.Cu) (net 2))
 (segment (start 123.893 61.7617) (end 124.722 60.9327) (width 0.75) (layer B.Cu) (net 2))
 (segment (start 124.722 60.9327) (end 125.095 60.9327) (width 0.75) (layer B.Cu) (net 2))
 (segment (start 125.095 60.9327) (end 125.095 59.6753) (width 0.75) (layer B.Cu) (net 2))
 (segment (start 125.095 58.15) (end 125.095 59.6753) (width 0.75) (layer B.Cu) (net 2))
 (segment (start 123.893 61.7617) (end 123.893 62.9485) (width 0.75) (layer B.Cu) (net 2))
 (segment (start 121.393 62.4481) (end 122.0794 61.7617) (width 0.75) (layer B.Cu) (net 2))
 (segment (start 122.0794 61.7617) (end 123.893 61.7617) (width 0.75) (layer B.Cu) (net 2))
 (segment (start 123.893 62.9485) (end 123.893 64.0715) (width 0.75) (layer B.Cu) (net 2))
 (segment (start 121.393 62.4481) (end 121.393 62.9485) (width 0.75) (layer B.Cu) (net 2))
 (segment (start 120.015 58.15) (end 120.015 59.6753) (width 0.75) (layer B.Cu) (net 2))
 (segment (start 114.2925 60.3178) (end 114.935 59.6753) (width 0.75) (layer B.Cu) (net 2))
 (segment (start 109.855 59.6753) (end 113.65 59.6753) (width 0.75) (layer B.Cu) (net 2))
 (segment (start 113.65 59.6753) (end 114.2925 60.3178) (width 0.75) (layer B.Cu) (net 2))
 (segment (start 104.775 58.15) (end 106.3003 59.6753) (width 0.75) (layer B.Cu) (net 2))
 (segment (start 106.3003 59.6753) (end 109.855 59.6753) (width 0.75) (layer B.Cu) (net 2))
 (segment (start 114.935 58.15) (end 114.935 59.6753) (width 0.75) (layer B.Cu) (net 2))
 (segment (start 109.855 58.15) (end 109.855 59.6753) (width 0.75) (layer B.Cu) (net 2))
 (segment (start 118.893 62.9485) (end 118.893 64.0715) (width 0.75) (layer B.Cu) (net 2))
 (segment (start 116.393 64.0715) (end 116.393 62.9485) (width 0.75) (layer B.Cu) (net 2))
 (segment (start 113.893 62.9485) (end 113.893 64.0715) (width 0.75) (layer B.Cu) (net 2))
 (segment (start 126.393 64.0715) (end 126.393 62.9485) (width 0.75) (layer F.Cu) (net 2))
 (segment (start 123.893 64.0715) (end 123.893 62.9485) (width 0.75) (layer F.Cu) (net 2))
 (segment (start 121.393 64.0715) (end 121.393 62.9485) (width 0.75) (layer F.Cu) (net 2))
 (segment (start 118.893 64.0715) (end 118.893 62.9485) (width 0.75) (layer F.Cu) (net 2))
 (segment (start 116.393 64.0715) (end 116.393 62.9485) (width 0.75) (layer F.Cu) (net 2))
 (segment (start 113.893 64.0715) (end 113.893 62.9485) (width 0.75) (layer F.Cu) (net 2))
 (segment (start 121.393 64.0715) (end 121.393 62.9485) (width 0.75) (layer B.Cu) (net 2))
 (segment (start 126.393 64.0715) (end 126.393 62.9485) (width 0.75) (layer B.Cu) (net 2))
 (segment (start 96.393 62.9485) (end 96.393 64.0715) (width 0.5) (layer F.Cu) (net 17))
 (segment (start 96.393 61.9402) (end 96.393 62.9485) (width 0.5) (layer B.Cu) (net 17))
 (segment (start 79.375 58.15) (end 82.1263 60.9013) (width 0.5) (layer B.Cu) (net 17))
 (segment (start 82.1263 60.9013) (end 95.4502 60.9013) (width 0.5) (layer B.Cu) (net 17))
 (segment (start 95.4502 60.9013) (end 96.393 61.8441) (width 0.5) (layer B.Cu) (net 17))
 (segment (start 96.393 61.8441) (end 96.393 61.9402) (width 0.5) (layer B.Cu) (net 17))
 (segment (start 98.893 62.6133) (end 98.2199 61.9402) (width 0.5) (layer B.Cu) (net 17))
 (segment (start 98.2199 61.9402) (end 96.393 61.9402) (width 0.5) (layer B.Cu) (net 17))
 (segment (start 98.893 62.6133) (end 98.893 62.9485) (width 0.5) (layer B.Cu) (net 17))
 (segment (start 101.393 62.9485) (end 101.393 62.6214) (width 0.5) (layer B.Cu) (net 17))
 (segment (start 101.393 62.6214) (end 100.6947 61.9231) (width 0.5) (layer B.Cu) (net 17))
 (segment (start 100.6947 61.9231) (end 99.5832 61.9231) (width 0.5) (layer B.Cu) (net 17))
 (segment (start 99.5832 61.9231) (end 98.893 62.6133) (width 0.5) (layer B.Cu) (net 17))
 (segment (start 74.295 56.7497) (end 77.9747 56.7497) (width 0.5) (layer B.Cu) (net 17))
 (segment (start 77.9747 56.7497) (end 79.375 58.15) (width 0.5) (layer B.Cu) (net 17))
 (segment (start 96.393 64.0715) (end 96.393 62.9485) (width 0.5) (layer B.Cu) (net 17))
 (segment (start 101.393 64.0715) (end 101.393 62.9485) (width 0.5) (layer F.Cu) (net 17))
 (segment (start 98.893 64.0715) (end 98.893 62.9485) (width 0.5) (layer F.Cu) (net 17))
 (segment (start 98.893 64.0715) (end 98.893 62.9485) (width 0.5) (layer B.Cu) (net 17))
 (segment (start 101.393 64.0715) (end 101.393 62.9485) (width 0.5) (layer B.Cu) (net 17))
 (segment (start 69.215 58.15) (end 70.6153 56.7497) (width 0.5) (layer B.Cu) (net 17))
 (segment (start 70.6153 56.7497) (end 74.295 56.7497) (width 0.5) (layer B.Cu) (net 17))
 (segment (start 74.295 58.15) (end 74.295 56.7497) (width 0.5) (layer B.Cu) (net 17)))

